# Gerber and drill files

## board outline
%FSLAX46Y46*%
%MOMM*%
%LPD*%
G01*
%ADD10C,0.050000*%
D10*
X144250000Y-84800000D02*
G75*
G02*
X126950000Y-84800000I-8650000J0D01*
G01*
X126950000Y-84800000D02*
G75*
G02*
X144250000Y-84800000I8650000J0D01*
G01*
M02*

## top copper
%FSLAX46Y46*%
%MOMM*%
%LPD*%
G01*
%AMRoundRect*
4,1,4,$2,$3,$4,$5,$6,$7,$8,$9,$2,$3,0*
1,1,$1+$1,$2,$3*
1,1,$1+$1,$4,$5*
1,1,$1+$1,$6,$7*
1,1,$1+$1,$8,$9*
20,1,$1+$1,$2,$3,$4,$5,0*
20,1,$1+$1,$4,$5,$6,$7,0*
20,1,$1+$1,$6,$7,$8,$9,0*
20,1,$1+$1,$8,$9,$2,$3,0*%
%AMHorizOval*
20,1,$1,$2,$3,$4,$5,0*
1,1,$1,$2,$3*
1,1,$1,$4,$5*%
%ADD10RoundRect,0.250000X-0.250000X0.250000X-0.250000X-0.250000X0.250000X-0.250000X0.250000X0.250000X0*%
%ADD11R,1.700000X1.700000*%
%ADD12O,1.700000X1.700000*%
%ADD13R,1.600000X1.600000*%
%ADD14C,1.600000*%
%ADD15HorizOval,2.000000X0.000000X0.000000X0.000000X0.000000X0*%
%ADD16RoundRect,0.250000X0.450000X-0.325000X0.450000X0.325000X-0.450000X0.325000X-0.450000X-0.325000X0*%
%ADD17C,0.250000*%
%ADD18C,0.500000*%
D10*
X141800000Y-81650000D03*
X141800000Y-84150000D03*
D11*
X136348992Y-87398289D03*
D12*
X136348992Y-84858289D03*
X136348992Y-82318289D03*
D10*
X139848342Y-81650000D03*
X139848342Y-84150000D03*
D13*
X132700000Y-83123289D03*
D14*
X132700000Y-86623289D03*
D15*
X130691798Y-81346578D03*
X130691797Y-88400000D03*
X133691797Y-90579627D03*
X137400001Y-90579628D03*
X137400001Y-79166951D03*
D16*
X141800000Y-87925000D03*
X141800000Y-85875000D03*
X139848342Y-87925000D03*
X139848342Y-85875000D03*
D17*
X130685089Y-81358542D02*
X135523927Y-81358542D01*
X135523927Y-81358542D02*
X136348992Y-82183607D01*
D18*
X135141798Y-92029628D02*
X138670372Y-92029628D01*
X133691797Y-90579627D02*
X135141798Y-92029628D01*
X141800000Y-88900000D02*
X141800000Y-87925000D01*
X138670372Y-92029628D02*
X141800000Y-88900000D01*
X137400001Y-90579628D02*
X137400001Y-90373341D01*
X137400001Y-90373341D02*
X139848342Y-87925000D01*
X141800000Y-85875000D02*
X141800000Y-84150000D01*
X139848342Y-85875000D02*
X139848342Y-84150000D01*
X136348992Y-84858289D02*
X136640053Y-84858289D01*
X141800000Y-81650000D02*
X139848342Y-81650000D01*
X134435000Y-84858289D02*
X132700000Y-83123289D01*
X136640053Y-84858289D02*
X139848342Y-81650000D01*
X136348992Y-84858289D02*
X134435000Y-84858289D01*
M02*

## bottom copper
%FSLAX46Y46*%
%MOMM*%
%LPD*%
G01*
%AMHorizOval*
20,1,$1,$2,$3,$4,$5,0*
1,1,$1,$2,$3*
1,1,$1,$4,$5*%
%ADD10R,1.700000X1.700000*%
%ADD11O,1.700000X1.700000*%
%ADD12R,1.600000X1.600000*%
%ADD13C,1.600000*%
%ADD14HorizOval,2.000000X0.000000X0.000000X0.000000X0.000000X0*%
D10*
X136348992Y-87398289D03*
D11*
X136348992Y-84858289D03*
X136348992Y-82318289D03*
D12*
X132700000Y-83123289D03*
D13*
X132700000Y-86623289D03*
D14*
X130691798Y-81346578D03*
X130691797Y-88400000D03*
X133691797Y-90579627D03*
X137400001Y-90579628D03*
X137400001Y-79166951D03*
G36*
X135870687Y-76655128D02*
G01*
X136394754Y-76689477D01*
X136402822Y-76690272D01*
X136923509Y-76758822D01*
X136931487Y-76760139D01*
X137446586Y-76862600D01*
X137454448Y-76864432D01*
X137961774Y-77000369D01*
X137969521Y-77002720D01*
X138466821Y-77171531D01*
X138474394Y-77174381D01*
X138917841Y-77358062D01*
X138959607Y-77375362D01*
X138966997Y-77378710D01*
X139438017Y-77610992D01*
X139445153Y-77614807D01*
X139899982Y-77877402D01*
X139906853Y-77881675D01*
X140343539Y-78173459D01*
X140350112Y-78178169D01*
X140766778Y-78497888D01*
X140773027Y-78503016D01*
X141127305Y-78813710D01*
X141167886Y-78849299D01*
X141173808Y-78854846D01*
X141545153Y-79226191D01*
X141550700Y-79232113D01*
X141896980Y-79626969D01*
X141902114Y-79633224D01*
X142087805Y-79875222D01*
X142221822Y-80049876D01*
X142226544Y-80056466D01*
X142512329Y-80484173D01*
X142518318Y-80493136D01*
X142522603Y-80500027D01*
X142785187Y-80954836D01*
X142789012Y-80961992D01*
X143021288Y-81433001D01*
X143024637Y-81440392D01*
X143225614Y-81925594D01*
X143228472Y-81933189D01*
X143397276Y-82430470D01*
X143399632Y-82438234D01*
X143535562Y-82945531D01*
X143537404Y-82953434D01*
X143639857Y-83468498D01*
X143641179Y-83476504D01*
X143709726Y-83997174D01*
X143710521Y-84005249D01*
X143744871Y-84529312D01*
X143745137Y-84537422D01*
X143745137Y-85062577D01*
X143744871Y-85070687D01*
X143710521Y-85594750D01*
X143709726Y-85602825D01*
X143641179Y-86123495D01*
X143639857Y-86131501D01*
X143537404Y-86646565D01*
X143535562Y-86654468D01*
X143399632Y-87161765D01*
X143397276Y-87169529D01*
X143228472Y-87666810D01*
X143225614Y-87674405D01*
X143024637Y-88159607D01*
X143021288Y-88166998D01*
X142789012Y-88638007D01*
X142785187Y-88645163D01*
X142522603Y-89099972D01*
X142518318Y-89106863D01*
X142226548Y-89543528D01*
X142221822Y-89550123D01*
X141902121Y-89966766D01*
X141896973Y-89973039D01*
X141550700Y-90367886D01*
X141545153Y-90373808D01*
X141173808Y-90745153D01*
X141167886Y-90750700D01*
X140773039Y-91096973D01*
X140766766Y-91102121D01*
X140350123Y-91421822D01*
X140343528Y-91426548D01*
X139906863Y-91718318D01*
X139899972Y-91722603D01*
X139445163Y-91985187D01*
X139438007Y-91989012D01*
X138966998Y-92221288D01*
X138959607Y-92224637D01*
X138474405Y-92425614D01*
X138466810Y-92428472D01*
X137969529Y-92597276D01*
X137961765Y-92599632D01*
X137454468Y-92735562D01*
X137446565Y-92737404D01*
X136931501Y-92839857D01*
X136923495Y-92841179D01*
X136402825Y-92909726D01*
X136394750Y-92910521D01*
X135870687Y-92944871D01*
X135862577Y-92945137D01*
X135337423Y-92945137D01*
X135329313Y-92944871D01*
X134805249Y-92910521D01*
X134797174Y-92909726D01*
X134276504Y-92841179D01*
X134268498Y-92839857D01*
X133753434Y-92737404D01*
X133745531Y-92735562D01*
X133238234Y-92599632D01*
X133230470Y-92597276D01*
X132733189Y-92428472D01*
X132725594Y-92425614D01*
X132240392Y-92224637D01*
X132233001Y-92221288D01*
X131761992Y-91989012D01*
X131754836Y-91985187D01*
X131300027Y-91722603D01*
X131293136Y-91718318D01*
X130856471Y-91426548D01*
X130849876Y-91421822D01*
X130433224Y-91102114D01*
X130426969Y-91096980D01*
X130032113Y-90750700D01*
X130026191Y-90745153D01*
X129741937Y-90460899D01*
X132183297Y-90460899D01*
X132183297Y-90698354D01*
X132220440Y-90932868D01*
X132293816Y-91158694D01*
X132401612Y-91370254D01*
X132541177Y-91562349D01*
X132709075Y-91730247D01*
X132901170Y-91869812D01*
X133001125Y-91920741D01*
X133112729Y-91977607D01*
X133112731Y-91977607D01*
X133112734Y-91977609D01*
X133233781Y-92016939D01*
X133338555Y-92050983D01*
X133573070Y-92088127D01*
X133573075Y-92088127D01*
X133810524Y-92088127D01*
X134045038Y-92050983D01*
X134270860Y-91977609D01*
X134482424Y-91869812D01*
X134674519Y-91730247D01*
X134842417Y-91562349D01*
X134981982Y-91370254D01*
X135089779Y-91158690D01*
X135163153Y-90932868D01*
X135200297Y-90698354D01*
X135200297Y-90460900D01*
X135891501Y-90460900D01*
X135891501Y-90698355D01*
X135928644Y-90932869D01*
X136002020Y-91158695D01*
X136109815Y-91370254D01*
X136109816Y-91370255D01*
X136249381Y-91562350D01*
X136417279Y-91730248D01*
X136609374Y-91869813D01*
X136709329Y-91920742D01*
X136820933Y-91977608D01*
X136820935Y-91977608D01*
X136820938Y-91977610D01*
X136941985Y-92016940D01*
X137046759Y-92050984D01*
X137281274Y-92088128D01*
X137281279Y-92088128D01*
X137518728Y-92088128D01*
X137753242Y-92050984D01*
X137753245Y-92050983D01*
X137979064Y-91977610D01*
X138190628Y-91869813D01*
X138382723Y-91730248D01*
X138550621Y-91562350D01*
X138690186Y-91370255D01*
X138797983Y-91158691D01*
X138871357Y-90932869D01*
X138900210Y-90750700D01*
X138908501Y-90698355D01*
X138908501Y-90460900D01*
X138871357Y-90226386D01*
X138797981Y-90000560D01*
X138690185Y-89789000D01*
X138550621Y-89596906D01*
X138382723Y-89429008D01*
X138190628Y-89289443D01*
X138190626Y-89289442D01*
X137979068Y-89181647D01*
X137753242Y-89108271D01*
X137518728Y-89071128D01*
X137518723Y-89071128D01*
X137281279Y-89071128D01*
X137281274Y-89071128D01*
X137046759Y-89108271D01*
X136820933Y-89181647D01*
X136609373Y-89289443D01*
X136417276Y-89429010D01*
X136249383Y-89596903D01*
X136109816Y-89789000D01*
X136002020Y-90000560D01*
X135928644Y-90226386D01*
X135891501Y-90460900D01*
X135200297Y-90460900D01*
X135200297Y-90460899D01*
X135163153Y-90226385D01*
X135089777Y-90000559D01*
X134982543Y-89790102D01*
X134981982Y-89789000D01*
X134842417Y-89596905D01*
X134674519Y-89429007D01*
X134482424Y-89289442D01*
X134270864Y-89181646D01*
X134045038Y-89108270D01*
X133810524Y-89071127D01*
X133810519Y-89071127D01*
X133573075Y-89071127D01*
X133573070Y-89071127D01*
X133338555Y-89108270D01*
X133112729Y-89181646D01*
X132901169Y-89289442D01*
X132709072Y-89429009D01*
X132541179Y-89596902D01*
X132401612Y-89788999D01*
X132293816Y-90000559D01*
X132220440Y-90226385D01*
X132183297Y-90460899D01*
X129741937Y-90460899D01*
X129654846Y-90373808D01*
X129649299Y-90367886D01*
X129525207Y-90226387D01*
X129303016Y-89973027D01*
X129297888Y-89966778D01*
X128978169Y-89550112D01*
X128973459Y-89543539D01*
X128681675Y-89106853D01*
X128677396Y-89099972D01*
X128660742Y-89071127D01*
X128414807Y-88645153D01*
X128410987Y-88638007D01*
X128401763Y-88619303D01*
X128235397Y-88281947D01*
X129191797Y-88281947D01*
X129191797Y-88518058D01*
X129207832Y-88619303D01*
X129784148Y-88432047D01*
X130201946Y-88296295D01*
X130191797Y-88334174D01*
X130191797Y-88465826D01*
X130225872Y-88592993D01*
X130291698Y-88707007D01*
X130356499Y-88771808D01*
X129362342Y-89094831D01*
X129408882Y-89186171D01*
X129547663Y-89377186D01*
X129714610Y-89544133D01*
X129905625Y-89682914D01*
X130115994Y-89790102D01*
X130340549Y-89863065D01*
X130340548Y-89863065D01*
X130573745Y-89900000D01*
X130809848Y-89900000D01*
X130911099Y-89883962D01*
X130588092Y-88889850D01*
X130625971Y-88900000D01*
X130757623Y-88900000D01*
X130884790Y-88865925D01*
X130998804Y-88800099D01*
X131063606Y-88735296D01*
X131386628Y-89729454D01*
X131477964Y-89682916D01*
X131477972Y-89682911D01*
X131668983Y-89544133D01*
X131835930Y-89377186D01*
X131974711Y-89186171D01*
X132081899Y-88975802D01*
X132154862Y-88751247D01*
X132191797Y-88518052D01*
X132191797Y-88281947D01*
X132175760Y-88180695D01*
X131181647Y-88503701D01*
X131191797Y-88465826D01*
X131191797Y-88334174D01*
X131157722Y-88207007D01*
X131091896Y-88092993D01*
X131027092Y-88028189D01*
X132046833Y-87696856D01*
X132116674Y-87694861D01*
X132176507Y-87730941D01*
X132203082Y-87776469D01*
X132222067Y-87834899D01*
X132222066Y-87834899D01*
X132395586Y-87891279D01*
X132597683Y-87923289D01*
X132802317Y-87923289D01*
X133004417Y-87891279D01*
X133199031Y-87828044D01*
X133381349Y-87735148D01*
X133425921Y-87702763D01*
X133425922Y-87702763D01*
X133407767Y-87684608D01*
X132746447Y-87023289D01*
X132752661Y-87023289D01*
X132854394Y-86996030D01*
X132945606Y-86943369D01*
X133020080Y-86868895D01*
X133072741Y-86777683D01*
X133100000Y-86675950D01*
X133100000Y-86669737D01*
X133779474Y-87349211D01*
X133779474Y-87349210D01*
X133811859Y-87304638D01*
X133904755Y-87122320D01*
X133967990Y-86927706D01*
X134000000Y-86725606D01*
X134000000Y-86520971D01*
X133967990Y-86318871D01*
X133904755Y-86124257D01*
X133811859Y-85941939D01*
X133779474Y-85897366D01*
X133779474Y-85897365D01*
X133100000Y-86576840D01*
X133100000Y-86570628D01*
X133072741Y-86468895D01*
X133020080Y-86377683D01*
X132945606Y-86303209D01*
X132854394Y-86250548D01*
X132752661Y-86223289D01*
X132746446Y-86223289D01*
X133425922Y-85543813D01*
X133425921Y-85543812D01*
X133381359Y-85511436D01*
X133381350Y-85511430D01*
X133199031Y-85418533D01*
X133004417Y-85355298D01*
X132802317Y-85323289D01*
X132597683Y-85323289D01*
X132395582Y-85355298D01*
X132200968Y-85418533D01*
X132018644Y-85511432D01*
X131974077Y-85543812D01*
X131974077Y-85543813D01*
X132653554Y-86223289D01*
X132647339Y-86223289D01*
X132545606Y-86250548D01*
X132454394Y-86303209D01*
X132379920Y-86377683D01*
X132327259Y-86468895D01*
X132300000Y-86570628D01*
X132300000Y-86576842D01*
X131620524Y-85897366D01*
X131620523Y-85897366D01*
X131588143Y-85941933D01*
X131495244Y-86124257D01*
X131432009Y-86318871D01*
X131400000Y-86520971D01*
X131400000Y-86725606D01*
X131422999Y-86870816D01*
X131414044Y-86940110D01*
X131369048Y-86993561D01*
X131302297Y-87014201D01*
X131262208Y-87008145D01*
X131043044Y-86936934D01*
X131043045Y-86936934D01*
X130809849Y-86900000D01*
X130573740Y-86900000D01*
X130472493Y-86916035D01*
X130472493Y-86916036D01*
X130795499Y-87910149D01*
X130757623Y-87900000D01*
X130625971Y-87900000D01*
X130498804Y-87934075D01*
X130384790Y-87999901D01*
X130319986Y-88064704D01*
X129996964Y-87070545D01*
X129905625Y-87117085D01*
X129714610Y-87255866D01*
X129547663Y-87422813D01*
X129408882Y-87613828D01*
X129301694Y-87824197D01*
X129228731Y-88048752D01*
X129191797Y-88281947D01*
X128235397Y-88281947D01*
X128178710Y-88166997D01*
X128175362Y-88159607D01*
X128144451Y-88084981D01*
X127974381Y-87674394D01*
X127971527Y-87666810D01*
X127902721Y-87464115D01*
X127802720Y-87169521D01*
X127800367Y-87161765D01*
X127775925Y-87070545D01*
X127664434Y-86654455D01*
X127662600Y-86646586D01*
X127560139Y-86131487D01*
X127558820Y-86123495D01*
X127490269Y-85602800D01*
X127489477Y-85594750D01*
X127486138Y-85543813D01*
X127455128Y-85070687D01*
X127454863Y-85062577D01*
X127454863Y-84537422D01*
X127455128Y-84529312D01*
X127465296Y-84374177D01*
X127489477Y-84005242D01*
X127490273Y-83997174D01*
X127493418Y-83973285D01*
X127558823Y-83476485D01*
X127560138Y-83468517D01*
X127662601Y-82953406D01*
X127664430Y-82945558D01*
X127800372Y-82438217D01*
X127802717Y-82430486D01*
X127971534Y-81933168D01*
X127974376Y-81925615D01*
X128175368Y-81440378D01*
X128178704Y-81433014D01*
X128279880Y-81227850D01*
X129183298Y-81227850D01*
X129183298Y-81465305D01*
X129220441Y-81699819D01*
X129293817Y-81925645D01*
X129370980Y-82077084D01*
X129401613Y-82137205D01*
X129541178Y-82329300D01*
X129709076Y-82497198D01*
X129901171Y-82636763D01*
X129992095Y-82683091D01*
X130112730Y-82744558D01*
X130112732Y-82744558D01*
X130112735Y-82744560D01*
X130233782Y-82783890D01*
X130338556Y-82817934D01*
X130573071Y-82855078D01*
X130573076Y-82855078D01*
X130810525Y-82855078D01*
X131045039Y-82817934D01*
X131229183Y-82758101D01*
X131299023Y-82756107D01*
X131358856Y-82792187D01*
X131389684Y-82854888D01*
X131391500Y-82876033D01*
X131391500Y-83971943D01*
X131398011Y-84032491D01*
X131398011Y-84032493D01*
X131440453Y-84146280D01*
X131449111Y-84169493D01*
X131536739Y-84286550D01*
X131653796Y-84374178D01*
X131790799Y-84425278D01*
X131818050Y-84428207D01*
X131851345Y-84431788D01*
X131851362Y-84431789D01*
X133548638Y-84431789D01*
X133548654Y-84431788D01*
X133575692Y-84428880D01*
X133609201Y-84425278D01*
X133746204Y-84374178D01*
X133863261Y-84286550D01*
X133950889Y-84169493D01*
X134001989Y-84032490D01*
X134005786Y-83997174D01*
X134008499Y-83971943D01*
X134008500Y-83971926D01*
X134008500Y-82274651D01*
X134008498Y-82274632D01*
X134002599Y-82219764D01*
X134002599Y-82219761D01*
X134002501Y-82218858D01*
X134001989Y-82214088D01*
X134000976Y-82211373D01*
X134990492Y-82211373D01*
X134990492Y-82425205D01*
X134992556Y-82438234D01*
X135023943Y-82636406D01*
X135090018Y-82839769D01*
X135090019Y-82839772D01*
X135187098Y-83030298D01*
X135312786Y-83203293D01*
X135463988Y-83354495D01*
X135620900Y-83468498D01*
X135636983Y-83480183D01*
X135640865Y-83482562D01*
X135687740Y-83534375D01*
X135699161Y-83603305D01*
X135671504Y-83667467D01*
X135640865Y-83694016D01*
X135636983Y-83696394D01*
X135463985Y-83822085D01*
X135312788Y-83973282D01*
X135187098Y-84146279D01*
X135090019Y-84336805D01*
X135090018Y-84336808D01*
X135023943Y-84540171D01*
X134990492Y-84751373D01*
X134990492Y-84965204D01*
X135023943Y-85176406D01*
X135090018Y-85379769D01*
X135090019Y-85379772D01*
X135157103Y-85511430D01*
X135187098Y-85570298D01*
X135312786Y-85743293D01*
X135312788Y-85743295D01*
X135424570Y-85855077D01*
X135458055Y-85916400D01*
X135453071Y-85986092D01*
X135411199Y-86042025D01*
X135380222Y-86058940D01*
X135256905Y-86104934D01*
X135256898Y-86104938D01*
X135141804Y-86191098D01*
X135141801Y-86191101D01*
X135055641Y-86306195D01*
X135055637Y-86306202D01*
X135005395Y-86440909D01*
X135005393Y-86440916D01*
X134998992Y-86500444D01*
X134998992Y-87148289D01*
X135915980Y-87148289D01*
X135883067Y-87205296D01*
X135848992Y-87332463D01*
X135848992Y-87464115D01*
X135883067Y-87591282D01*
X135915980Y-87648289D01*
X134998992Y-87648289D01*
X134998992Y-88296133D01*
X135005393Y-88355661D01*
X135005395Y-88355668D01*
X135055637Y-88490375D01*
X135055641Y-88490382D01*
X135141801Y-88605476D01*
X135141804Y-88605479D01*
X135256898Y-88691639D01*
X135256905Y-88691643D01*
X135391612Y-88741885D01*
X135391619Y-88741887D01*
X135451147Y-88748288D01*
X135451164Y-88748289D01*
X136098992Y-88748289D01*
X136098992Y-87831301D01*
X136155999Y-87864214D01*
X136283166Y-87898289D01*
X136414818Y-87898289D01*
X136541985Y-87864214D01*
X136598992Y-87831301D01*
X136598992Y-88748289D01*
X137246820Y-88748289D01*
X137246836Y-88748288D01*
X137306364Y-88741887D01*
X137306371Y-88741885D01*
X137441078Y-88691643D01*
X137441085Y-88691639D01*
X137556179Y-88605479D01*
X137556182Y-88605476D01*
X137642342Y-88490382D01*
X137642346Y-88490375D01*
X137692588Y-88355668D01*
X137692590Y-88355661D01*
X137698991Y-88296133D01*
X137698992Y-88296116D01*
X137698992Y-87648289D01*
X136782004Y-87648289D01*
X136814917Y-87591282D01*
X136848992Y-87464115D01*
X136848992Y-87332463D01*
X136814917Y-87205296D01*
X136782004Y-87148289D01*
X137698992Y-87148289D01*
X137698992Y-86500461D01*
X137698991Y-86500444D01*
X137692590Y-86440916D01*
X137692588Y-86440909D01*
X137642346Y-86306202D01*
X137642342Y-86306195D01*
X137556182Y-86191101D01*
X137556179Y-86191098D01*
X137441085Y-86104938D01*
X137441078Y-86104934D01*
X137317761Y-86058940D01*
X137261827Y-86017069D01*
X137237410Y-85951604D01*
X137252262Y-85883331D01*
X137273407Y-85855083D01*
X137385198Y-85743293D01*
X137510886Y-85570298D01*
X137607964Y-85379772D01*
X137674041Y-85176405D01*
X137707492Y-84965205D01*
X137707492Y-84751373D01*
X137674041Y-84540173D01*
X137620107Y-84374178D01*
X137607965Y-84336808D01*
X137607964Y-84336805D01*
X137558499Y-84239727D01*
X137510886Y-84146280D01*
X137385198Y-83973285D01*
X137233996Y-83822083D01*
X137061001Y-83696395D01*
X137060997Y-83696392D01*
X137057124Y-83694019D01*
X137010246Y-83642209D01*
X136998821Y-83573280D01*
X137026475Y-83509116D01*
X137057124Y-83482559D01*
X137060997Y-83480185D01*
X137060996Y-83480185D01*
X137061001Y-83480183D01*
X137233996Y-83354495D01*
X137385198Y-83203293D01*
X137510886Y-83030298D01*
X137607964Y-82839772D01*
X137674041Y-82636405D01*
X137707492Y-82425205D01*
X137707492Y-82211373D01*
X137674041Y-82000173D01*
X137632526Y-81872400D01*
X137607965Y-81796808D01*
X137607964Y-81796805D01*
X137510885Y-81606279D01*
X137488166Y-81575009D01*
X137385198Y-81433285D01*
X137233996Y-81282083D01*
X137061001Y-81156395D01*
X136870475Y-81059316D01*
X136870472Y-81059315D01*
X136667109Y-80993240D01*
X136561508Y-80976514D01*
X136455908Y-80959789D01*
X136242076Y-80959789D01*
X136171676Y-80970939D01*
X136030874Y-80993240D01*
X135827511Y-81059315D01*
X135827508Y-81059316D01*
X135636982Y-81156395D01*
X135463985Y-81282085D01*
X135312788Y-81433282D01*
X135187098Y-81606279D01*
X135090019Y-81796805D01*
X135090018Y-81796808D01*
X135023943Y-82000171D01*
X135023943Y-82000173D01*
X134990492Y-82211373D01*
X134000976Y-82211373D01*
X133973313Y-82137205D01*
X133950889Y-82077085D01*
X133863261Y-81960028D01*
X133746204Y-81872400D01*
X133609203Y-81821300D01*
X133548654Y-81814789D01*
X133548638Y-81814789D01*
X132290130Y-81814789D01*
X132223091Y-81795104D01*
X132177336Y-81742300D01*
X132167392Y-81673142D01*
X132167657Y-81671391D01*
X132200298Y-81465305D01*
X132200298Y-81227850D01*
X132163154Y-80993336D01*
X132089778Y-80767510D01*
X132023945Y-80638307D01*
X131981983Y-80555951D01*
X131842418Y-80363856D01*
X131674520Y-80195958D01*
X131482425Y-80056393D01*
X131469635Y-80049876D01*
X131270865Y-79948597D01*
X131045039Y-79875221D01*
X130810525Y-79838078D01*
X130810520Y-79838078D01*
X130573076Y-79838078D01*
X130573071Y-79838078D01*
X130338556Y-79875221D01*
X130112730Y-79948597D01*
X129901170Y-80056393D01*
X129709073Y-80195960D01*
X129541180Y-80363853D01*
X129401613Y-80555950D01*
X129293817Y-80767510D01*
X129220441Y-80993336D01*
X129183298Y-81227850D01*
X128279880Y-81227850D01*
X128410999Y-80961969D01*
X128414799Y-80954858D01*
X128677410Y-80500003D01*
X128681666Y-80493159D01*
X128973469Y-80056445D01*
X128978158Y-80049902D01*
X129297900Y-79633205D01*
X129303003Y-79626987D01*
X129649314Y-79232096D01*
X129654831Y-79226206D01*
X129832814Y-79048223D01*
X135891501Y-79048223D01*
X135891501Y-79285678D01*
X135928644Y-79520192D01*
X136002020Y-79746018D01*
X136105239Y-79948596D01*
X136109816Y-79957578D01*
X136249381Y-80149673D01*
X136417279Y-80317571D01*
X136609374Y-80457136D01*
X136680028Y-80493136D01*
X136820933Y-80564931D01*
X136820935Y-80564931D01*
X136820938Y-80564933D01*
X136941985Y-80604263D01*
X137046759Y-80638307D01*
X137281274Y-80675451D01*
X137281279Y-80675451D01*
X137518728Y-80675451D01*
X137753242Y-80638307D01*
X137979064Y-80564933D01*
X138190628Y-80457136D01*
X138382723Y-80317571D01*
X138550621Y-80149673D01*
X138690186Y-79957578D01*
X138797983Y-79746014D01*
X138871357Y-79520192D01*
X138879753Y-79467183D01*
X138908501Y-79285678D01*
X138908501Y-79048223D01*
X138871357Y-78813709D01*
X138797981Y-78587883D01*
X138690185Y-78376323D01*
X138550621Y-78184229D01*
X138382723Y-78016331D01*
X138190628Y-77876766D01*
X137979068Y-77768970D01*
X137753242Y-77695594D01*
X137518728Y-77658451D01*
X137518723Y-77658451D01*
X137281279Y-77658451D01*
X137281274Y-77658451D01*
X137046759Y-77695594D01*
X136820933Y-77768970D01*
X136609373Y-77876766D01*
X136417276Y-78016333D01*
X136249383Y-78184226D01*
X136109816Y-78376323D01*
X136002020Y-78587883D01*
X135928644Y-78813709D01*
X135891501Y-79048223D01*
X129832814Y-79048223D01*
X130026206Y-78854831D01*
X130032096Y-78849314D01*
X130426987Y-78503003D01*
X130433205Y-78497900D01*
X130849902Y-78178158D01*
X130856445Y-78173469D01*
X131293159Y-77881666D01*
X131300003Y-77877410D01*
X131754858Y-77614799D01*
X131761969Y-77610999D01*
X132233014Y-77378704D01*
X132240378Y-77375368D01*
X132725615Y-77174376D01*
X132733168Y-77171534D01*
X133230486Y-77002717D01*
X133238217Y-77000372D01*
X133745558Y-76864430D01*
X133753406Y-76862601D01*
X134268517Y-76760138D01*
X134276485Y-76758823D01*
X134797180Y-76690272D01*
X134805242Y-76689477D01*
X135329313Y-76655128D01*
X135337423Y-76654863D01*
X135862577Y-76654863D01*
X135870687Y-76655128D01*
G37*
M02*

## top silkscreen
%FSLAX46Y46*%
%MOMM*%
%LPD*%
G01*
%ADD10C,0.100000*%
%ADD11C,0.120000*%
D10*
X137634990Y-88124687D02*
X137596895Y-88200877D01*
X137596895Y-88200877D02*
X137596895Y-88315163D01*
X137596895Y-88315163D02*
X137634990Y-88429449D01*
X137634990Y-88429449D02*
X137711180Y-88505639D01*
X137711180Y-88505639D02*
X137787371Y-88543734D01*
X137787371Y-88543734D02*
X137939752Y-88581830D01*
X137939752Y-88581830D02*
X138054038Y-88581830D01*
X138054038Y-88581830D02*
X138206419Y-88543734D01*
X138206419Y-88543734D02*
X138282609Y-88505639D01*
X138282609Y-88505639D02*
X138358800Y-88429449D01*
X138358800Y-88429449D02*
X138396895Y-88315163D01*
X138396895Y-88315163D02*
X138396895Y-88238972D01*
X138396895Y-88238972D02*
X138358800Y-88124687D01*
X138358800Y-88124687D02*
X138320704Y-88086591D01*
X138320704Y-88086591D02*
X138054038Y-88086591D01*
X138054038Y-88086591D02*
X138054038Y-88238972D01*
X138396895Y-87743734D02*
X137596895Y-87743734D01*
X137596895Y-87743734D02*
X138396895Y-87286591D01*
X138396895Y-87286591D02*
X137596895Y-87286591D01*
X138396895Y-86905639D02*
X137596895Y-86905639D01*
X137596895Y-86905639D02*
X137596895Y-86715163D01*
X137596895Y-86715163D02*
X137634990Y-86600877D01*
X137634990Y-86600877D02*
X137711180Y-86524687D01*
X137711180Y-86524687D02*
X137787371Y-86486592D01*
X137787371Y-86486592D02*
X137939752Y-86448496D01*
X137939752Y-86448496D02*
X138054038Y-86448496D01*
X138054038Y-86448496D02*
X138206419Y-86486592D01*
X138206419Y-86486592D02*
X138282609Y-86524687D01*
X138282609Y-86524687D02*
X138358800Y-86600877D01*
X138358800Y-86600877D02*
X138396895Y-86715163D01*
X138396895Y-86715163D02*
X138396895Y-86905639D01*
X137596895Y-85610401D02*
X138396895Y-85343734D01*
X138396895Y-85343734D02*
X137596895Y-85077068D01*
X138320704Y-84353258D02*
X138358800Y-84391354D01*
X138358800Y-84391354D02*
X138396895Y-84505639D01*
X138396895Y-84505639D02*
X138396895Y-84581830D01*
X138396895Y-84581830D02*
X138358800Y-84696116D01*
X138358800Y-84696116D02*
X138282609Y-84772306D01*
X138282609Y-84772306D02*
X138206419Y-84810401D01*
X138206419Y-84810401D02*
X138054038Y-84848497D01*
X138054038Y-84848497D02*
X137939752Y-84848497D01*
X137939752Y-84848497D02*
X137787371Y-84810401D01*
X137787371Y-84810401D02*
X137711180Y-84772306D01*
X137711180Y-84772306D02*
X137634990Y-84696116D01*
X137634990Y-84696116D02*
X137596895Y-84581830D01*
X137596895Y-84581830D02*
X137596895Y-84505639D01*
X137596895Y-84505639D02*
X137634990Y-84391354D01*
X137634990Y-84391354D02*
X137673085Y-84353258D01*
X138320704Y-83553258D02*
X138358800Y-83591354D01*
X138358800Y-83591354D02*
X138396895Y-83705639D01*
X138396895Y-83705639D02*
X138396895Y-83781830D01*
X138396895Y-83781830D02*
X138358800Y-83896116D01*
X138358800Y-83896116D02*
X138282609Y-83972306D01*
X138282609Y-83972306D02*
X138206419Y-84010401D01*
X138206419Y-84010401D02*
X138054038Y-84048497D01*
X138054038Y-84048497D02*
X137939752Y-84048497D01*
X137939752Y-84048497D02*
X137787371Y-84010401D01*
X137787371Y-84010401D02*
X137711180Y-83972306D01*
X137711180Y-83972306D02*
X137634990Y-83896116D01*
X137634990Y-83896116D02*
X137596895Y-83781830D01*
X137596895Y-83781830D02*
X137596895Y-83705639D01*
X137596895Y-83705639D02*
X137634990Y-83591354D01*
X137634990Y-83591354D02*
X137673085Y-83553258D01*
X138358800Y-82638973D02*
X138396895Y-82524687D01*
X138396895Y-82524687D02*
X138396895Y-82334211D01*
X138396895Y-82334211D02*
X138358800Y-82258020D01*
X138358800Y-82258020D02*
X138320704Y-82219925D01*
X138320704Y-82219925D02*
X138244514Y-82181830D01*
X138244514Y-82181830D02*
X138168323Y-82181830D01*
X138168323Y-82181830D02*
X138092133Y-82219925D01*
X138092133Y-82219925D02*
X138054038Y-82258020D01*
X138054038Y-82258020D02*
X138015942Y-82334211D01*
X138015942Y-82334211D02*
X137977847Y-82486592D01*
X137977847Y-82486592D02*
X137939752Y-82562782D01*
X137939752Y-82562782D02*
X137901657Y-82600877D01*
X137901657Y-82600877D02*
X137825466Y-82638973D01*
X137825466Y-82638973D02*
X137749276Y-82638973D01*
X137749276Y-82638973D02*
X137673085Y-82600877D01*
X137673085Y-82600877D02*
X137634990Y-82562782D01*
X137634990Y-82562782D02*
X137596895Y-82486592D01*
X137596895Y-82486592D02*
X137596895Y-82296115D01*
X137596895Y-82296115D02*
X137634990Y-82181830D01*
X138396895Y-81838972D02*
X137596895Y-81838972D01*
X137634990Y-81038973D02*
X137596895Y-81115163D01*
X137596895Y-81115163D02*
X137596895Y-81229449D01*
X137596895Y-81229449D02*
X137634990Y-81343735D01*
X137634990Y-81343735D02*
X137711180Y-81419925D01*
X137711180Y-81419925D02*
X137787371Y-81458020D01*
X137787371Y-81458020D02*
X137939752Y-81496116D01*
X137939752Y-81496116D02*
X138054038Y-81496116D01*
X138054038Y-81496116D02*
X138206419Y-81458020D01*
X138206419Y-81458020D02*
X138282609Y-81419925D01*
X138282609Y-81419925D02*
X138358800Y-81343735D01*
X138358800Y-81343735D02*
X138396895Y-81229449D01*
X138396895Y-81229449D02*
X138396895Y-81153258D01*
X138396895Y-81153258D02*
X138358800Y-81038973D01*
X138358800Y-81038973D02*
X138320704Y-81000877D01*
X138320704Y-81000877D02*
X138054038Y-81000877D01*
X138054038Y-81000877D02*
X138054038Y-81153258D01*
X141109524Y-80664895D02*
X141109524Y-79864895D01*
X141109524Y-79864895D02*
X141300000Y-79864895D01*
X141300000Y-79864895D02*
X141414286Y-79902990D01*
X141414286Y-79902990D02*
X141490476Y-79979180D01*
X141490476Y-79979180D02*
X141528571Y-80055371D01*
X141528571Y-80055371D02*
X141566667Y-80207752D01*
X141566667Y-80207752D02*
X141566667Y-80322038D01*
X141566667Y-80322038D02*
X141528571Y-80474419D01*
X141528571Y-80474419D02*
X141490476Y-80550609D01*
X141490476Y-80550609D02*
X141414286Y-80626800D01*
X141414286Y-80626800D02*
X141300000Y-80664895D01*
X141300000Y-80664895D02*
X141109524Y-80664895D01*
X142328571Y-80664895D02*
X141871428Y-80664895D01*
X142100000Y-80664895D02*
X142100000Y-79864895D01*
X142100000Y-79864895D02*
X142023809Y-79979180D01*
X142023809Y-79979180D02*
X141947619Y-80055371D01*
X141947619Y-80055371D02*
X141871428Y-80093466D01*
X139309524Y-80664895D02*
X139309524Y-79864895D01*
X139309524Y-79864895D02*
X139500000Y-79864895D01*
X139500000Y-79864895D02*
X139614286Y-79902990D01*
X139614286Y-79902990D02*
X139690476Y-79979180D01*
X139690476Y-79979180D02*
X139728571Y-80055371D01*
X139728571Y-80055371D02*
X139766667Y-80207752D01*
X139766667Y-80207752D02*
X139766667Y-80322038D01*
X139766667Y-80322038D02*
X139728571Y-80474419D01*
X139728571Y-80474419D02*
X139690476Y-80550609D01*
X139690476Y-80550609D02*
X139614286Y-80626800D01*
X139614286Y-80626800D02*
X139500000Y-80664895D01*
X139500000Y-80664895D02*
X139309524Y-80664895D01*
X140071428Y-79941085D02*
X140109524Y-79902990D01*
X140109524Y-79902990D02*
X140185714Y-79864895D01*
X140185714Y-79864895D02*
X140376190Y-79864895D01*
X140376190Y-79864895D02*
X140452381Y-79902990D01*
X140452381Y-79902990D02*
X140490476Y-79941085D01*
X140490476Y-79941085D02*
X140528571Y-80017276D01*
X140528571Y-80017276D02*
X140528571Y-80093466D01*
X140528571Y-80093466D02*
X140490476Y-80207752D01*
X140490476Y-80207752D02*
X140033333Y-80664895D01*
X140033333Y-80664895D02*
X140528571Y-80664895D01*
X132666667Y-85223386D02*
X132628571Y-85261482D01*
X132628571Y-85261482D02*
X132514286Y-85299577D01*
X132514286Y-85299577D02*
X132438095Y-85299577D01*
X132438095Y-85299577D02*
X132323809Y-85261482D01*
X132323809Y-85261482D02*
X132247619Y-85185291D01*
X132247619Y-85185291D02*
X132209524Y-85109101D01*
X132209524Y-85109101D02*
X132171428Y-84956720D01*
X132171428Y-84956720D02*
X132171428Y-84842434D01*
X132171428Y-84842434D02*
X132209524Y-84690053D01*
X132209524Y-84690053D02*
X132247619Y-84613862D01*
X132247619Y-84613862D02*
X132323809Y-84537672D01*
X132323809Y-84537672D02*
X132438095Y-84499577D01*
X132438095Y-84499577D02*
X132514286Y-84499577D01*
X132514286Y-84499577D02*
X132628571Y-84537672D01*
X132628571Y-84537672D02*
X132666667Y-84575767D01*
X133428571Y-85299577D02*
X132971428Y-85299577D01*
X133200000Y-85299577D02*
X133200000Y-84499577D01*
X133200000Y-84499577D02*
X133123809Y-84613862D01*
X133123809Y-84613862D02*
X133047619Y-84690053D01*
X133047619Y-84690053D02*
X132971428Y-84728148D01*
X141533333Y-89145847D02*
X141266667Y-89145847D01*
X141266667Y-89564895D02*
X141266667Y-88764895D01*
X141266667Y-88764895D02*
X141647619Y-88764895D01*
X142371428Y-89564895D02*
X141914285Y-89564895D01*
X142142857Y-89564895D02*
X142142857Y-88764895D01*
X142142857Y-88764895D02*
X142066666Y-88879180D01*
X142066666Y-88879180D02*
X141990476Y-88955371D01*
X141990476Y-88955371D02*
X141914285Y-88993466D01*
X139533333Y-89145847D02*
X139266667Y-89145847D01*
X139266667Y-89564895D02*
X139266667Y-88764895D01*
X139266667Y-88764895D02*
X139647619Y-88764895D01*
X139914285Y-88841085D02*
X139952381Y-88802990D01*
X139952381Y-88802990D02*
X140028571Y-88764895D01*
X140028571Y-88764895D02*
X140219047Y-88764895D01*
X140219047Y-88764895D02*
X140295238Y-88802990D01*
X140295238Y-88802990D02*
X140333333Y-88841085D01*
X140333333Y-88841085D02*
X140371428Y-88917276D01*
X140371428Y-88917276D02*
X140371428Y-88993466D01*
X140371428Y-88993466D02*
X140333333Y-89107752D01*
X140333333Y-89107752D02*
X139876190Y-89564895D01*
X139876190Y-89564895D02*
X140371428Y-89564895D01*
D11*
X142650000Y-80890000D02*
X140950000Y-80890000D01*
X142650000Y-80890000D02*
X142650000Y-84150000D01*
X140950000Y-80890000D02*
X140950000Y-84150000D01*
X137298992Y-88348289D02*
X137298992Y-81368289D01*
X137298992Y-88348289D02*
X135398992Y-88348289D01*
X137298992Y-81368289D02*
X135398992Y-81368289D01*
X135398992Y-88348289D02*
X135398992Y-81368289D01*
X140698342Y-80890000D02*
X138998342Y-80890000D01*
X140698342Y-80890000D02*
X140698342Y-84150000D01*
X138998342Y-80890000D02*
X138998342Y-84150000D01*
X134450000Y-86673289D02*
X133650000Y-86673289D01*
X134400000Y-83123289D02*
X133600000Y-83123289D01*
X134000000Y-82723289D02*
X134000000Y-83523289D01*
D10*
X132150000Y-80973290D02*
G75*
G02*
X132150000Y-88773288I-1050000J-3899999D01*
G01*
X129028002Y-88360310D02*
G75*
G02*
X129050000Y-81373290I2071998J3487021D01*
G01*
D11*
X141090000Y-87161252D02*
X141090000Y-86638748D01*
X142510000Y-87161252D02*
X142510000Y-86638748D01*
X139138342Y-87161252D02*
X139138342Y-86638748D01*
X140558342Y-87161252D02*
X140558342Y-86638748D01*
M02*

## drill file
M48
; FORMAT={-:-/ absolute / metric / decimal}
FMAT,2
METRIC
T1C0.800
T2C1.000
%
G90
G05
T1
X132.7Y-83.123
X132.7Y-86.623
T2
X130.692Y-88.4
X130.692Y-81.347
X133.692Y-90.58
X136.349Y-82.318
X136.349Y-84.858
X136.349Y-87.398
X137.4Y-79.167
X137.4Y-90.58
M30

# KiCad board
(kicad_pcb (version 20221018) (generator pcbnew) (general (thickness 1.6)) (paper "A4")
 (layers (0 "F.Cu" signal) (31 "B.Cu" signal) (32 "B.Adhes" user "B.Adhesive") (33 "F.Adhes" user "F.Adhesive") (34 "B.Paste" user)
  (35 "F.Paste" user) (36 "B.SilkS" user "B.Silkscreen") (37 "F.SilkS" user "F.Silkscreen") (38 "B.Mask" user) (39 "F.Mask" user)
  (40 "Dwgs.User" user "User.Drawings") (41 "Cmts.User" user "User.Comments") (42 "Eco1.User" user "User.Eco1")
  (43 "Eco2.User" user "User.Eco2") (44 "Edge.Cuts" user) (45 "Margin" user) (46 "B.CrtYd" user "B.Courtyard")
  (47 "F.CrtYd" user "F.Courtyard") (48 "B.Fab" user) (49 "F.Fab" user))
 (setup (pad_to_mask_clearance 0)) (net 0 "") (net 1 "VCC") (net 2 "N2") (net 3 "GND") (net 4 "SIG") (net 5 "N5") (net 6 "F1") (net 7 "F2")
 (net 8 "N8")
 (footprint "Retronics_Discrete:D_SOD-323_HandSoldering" (layer "F.Cu") (at 141.8 82.9 -90)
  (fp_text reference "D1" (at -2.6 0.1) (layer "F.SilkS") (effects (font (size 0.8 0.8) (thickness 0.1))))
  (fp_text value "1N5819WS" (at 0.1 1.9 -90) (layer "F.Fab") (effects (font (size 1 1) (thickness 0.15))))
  (fp_line (start -2.01 -0.85) (end -2.01 0.85) (stroke (width 0.12) (type solid)) (layer "F.SilkS"))
  (fp_line (start -2.01 -0.85) (end 1.25 -0.85) (stroke (width 0.12) (type solid)) (layer "F.SilkS"))
  (fp_line (start -2.01 0.85) (end 1.25 0.85) (stroke (width 0.12) (type solid)) (layer "F.SilkS"))
  (pad "1" smd roundrect (at -1.25 0 270) (size 1 1) (layers "F.Cu" "F.Paste" "F.Mask") (roundrect_rratio 0.25) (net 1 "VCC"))
  (pad "2" smd roundrect (at 1.25 0 270) (size 1 1) (layers "F.Cu" "F.Paste" "F.Mask") (roundrect_rratio 0.25) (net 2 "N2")))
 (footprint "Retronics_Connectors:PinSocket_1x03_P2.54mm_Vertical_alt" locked (layer "F.Cu") (at 136.348992 87.398289 180)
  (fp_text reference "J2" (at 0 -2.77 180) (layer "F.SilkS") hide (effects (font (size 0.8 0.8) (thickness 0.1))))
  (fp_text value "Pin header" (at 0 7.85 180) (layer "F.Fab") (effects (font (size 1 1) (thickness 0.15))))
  (fp_line (start -0.95 -0.95) (end -0.95 6.03) (stroke (width 0.12) (type solid)) (layer "F.SilkS"))
  (fp_line (start -0.95 -0.95) (end 0.95 -0.95) (stroke (width 0.12) (type solid)) (layer "F.SilkS"))
  (fp_line (start -0.95 6.03) (end 0.95 6.03) (stroke (width 0.12) (type solid)) (layer "F.SilkS"))
  (fp_line (start 0.95 -0.95) (end 0.95 6.03) (stroke (width 0.12) (type solid)) (layer "F.SilkS"))
  (pad "1" thru_hole rect locked (at 0 0 180) (size 1.7 1.7) (drill 1) (layers "*.Cu" "*.Mask") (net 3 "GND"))
  (pad "2" thru_hole oval locked (at 0 2.54 180) (size 1.7 1.7) (drill 1) (layers "*.Cu" "*.Mask") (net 1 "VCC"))
  (pad "3" thru_hole oval locked (at 0 5.08 180) (size 1.7 1.7) (drill 1) (layers "*.Cu" "*.Mask") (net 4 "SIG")))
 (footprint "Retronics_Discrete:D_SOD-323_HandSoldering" (layer "F.Cu") (at 139.848342 82.9 -90)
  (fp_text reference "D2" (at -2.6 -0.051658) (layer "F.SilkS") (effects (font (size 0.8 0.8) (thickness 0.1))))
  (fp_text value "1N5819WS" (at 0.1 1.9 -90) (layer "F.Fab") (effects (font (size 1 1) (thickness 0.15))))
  (fp_line (start -2.01 -0.85) (end -2.01 0.85) (stroke (width 0.12) (type solid)) (layer "F.SilkS"))
  (fp_line (start -2.01 -0.85) (end 1.25 -0.85) (stroke (width 0.12) (type solid)) (layer "F.SilkS"))
  (fp_line (start -2.01 0.85) (end 1.25 0.85) (stroke (width 0.12) (type solid)) (layer "F.SilkS"))
  (pad "1" smd roundrect (at -1.25 0 270) (size 1 1) (layers "F.Cu" "F.Paste" "F.Mask") (roundrect_rratio 0.25) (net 1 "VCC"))
  (pad "2" smd roundrect (at 1.25 0 270) (size 1 1) (layers "F.Cu" "F.Paste" "F.Mask") (roundrect_rratio 0.25) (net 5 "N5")))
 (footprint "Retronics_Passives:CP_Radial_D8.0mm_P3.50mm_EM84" (layer "F.Cu") (at 131.1 83.123289 180)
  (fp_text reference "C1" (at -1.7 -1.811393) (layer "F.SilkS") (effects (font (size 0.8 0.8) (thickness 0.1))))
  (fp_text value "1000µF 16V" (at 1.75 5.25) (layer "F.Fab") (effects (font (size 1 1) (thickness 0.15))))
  (fp_line (start -3.35 -3.55) (end -2.55 -3.55) (stroke (width 0.12) (type solid)) (layer "F.SilkS"))
  (fp_line (start -3.3 0) (end -2.5 0) (stroke (width 0.12) (type solid)) (layer "F.SilkS"))
  (fp_line (start -2.9 0.4) (end -2.9 -0.4) (stroke (width 0.12) (type solid)) (layer "F.SilkS"))
  (fp_arc (start -1.05 2.149999) (mid -4.038873 -1.75) (end -1.05 -5.649999) (stroke (width 0.1) (type default)) (layer "F.SilkS"))
  (fp_arc (start 2.071998 -5.237021) (mid 4.056147 -1.73723) (end 2.05 1.749999) (stroke (width 0.1) (type default)) (layer "F.SilkS"))
  (pad "1" thru_hole rect (at -1.6 0 270) (size 1.6 1.6) (drill 0.8) (layers "*.Cu" "*.Mask") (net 1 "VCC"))
  (pad "2" thru_hole circle (at -1.6 -3.5 270) (size 1.6 1.6) (drill 0.8) (layers "*.Cu" "*.Mask") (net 3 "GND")))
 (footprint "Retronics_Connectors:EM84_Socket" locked (layer "F.Cu") (at 135.545899 84.873289)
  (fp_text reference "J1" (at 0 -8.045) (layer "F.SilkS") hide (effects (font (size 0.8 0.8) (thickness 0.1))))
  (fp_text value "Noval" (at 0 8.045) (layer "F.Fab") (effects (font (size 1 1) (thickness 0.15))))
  (pad "1" thru_hole oval locked (at -4.854101 -3.526711 18) (size 2 2) (drill 1) (layers "*.Cu" "*.Mask") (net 4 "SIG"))
  (pad "3" thru_hole oval locked (at -4.854102 3.526711 18) (size 2 2) (drill 1) (layers "*.Cu" "*.Mask") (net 3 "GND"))
  (pad "4" thru_hole oval locked (at -1.854102 5.706338 18) (size 2 2) (drill 1) (layers "*.Cu" "*.Mask") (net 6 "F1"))
  (pad "5" thru_hole oval locked (at 1.854102 5.706339 18) (size 2 2) (drill 1) (layers "*.Cu" "*.Mask") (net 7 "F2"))
  (pad "9" thru_hole oval locked (at 1.854102 -5.706338 18) (size 2 2) (drill 1) (layers "*.Cu" "*.Mask") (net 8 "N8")))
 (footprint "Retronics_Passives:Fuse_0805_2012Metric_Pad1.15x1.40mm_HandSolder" (layer "F.Cu") (at 141.8 86.9 90)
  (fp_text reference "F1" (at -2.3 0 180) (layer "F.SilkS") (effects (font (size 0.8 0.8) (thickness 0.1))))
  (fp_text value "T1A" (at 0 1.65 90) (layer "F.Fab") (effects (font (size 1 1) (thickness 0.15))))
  (fp_line (start -0.261252 -0.71) (end 0.261252 -0.71) (stroke (width 0.12) (type solid)) (layer "F.SilkS"))
  (fp_line (start -0.261252 0.71) (end 0.261252 0.71) (stroke (width 0.12) (type solid)) (layer "F.SilkS"))
  (pad "1" smd roundrect (at -1.025 0 90) (size 1.15 1.4) (layers "F.Cu" "F.Paste" "F.Mask") (roundrect_rratio 0.2173913043) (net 6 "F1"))
  (pad "2" smd roundrect (at 1.025 0 90) (size 1.15 1.4) (layers "F.Cu" "F.Paste" "F.Mask") (roundrect_rratio 0.2173913043) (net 2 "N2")))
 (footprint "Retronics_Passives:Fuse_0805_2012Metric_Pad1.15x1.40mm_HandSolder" (layer "F.Cu") (at 139.848342 86.9 90)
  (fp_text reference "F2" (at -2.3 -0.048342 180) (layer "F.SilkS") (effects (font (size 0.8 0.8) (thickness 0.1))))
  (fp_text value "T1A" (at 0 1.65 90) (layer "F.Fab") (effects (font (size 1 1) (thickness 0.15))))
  (fp_line (start -0.261252 -0.71) (end 0.261252 -0.71) (stroke (width 0.12) (type solid)) (layer "F.SilkS"))
  (fp_line (start -0.261252 0.71) (end 0.261252 0.71) (stroke (width 0.12) (type solid)) (layer "F.SilkS"))
  (pad "1" smd roundrect (at -1.025 0 90) (size 1.15 1.4) (layers "F.Cu" "F.Paste" "F.Mask") (roundrect_rratio 0.2173913043) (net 7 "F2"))
  (pad "2" smd roundrect (at 1.025 0 90) (size 1.15 1.4) (layers "F.Cu" "F.Paste" "F.Mask") (roundrect_rratio 0.2173913043) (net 5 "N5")))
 (gr_circle (center 135.6 84.8) (end 143.778736 81.983835) (stroke (width 0.05) (type solid)) (fill none) (layer "Edge.Cuts"))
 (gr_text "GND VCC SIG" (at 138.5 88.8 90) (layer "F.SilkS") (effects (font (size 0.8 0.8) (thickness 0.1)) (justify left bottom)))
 (segment (start 130.685089 81.358542) (end 135.523927 81.358542) (width 0.25) (layer "F.Cu") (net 4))
 (segment (start 135.523927 81.358542) (end 136.348992 82.183607) (width 0.25) (layer "F.Cu") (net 4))
 (segment (start 135.141798 92.029628) (end 138.670372 92.029628) (width 0.5) (layer "F.Cu") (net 6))
 (segment (start 133.691797 90.579627) (end 135.141798 92.029628) (width 0.5) (layer "F.Cu") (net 6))
 (segment (start 141.8 88.9) (end 141.8 87.925) (width 0.5) (layer "F.Cu") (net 6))
 (segment (start 138.670372 92.029628) (end 141.8 88.9) (width 0.5) (layer "F.Cu") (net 6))
 (segment (start 137.400001 90.579628) (end 137.400001 90.373341) (width 0.5) (layer "F.Cu") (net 7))
 (segment (start 137.400001 90.373341) (end 139.848342 87.925) (width 0.5) (layer "F.Cu") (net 7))
 (segment (start 141.8 85.875) (end 141.8 84.15) (width 0.5) (layer "F.Cu") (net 2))
 (segment (start 139.848342 85.875) (end 139.848342 84.15) (width 0.5) (layer "F.Cu") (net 5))
 (segment (start 136.348992 84.858289) (end 136.640053 84.858289) (width 0.5) (layer "F.Cu") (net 1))
 (segment (start 141.8 81.65) (end 139.848342 81.65) (width 0.5) (layer "F.Cu") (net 1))
 (segment (start 134.435 84.858289) (end 132.7 83.123289) (width 0.5) (layer "F.Cu") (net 1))
 (segment (start 136.640053 84.858289) (end 139.848342 81.65) (width 0.5) (layer "F.Cu") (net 1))
 (segment (start 136.348992 84.858289) (end 134.435 84.858289) (width 0.5) (layer "F.Cu") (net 1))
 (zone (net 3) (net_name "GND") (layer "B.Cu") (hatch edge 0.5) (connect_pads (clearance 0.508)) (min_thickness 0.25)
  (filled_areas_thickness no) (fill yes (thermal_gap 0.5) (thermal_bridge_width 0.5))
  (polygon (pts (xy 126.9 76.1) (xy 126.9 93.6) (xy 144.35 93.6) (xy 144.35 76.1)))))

